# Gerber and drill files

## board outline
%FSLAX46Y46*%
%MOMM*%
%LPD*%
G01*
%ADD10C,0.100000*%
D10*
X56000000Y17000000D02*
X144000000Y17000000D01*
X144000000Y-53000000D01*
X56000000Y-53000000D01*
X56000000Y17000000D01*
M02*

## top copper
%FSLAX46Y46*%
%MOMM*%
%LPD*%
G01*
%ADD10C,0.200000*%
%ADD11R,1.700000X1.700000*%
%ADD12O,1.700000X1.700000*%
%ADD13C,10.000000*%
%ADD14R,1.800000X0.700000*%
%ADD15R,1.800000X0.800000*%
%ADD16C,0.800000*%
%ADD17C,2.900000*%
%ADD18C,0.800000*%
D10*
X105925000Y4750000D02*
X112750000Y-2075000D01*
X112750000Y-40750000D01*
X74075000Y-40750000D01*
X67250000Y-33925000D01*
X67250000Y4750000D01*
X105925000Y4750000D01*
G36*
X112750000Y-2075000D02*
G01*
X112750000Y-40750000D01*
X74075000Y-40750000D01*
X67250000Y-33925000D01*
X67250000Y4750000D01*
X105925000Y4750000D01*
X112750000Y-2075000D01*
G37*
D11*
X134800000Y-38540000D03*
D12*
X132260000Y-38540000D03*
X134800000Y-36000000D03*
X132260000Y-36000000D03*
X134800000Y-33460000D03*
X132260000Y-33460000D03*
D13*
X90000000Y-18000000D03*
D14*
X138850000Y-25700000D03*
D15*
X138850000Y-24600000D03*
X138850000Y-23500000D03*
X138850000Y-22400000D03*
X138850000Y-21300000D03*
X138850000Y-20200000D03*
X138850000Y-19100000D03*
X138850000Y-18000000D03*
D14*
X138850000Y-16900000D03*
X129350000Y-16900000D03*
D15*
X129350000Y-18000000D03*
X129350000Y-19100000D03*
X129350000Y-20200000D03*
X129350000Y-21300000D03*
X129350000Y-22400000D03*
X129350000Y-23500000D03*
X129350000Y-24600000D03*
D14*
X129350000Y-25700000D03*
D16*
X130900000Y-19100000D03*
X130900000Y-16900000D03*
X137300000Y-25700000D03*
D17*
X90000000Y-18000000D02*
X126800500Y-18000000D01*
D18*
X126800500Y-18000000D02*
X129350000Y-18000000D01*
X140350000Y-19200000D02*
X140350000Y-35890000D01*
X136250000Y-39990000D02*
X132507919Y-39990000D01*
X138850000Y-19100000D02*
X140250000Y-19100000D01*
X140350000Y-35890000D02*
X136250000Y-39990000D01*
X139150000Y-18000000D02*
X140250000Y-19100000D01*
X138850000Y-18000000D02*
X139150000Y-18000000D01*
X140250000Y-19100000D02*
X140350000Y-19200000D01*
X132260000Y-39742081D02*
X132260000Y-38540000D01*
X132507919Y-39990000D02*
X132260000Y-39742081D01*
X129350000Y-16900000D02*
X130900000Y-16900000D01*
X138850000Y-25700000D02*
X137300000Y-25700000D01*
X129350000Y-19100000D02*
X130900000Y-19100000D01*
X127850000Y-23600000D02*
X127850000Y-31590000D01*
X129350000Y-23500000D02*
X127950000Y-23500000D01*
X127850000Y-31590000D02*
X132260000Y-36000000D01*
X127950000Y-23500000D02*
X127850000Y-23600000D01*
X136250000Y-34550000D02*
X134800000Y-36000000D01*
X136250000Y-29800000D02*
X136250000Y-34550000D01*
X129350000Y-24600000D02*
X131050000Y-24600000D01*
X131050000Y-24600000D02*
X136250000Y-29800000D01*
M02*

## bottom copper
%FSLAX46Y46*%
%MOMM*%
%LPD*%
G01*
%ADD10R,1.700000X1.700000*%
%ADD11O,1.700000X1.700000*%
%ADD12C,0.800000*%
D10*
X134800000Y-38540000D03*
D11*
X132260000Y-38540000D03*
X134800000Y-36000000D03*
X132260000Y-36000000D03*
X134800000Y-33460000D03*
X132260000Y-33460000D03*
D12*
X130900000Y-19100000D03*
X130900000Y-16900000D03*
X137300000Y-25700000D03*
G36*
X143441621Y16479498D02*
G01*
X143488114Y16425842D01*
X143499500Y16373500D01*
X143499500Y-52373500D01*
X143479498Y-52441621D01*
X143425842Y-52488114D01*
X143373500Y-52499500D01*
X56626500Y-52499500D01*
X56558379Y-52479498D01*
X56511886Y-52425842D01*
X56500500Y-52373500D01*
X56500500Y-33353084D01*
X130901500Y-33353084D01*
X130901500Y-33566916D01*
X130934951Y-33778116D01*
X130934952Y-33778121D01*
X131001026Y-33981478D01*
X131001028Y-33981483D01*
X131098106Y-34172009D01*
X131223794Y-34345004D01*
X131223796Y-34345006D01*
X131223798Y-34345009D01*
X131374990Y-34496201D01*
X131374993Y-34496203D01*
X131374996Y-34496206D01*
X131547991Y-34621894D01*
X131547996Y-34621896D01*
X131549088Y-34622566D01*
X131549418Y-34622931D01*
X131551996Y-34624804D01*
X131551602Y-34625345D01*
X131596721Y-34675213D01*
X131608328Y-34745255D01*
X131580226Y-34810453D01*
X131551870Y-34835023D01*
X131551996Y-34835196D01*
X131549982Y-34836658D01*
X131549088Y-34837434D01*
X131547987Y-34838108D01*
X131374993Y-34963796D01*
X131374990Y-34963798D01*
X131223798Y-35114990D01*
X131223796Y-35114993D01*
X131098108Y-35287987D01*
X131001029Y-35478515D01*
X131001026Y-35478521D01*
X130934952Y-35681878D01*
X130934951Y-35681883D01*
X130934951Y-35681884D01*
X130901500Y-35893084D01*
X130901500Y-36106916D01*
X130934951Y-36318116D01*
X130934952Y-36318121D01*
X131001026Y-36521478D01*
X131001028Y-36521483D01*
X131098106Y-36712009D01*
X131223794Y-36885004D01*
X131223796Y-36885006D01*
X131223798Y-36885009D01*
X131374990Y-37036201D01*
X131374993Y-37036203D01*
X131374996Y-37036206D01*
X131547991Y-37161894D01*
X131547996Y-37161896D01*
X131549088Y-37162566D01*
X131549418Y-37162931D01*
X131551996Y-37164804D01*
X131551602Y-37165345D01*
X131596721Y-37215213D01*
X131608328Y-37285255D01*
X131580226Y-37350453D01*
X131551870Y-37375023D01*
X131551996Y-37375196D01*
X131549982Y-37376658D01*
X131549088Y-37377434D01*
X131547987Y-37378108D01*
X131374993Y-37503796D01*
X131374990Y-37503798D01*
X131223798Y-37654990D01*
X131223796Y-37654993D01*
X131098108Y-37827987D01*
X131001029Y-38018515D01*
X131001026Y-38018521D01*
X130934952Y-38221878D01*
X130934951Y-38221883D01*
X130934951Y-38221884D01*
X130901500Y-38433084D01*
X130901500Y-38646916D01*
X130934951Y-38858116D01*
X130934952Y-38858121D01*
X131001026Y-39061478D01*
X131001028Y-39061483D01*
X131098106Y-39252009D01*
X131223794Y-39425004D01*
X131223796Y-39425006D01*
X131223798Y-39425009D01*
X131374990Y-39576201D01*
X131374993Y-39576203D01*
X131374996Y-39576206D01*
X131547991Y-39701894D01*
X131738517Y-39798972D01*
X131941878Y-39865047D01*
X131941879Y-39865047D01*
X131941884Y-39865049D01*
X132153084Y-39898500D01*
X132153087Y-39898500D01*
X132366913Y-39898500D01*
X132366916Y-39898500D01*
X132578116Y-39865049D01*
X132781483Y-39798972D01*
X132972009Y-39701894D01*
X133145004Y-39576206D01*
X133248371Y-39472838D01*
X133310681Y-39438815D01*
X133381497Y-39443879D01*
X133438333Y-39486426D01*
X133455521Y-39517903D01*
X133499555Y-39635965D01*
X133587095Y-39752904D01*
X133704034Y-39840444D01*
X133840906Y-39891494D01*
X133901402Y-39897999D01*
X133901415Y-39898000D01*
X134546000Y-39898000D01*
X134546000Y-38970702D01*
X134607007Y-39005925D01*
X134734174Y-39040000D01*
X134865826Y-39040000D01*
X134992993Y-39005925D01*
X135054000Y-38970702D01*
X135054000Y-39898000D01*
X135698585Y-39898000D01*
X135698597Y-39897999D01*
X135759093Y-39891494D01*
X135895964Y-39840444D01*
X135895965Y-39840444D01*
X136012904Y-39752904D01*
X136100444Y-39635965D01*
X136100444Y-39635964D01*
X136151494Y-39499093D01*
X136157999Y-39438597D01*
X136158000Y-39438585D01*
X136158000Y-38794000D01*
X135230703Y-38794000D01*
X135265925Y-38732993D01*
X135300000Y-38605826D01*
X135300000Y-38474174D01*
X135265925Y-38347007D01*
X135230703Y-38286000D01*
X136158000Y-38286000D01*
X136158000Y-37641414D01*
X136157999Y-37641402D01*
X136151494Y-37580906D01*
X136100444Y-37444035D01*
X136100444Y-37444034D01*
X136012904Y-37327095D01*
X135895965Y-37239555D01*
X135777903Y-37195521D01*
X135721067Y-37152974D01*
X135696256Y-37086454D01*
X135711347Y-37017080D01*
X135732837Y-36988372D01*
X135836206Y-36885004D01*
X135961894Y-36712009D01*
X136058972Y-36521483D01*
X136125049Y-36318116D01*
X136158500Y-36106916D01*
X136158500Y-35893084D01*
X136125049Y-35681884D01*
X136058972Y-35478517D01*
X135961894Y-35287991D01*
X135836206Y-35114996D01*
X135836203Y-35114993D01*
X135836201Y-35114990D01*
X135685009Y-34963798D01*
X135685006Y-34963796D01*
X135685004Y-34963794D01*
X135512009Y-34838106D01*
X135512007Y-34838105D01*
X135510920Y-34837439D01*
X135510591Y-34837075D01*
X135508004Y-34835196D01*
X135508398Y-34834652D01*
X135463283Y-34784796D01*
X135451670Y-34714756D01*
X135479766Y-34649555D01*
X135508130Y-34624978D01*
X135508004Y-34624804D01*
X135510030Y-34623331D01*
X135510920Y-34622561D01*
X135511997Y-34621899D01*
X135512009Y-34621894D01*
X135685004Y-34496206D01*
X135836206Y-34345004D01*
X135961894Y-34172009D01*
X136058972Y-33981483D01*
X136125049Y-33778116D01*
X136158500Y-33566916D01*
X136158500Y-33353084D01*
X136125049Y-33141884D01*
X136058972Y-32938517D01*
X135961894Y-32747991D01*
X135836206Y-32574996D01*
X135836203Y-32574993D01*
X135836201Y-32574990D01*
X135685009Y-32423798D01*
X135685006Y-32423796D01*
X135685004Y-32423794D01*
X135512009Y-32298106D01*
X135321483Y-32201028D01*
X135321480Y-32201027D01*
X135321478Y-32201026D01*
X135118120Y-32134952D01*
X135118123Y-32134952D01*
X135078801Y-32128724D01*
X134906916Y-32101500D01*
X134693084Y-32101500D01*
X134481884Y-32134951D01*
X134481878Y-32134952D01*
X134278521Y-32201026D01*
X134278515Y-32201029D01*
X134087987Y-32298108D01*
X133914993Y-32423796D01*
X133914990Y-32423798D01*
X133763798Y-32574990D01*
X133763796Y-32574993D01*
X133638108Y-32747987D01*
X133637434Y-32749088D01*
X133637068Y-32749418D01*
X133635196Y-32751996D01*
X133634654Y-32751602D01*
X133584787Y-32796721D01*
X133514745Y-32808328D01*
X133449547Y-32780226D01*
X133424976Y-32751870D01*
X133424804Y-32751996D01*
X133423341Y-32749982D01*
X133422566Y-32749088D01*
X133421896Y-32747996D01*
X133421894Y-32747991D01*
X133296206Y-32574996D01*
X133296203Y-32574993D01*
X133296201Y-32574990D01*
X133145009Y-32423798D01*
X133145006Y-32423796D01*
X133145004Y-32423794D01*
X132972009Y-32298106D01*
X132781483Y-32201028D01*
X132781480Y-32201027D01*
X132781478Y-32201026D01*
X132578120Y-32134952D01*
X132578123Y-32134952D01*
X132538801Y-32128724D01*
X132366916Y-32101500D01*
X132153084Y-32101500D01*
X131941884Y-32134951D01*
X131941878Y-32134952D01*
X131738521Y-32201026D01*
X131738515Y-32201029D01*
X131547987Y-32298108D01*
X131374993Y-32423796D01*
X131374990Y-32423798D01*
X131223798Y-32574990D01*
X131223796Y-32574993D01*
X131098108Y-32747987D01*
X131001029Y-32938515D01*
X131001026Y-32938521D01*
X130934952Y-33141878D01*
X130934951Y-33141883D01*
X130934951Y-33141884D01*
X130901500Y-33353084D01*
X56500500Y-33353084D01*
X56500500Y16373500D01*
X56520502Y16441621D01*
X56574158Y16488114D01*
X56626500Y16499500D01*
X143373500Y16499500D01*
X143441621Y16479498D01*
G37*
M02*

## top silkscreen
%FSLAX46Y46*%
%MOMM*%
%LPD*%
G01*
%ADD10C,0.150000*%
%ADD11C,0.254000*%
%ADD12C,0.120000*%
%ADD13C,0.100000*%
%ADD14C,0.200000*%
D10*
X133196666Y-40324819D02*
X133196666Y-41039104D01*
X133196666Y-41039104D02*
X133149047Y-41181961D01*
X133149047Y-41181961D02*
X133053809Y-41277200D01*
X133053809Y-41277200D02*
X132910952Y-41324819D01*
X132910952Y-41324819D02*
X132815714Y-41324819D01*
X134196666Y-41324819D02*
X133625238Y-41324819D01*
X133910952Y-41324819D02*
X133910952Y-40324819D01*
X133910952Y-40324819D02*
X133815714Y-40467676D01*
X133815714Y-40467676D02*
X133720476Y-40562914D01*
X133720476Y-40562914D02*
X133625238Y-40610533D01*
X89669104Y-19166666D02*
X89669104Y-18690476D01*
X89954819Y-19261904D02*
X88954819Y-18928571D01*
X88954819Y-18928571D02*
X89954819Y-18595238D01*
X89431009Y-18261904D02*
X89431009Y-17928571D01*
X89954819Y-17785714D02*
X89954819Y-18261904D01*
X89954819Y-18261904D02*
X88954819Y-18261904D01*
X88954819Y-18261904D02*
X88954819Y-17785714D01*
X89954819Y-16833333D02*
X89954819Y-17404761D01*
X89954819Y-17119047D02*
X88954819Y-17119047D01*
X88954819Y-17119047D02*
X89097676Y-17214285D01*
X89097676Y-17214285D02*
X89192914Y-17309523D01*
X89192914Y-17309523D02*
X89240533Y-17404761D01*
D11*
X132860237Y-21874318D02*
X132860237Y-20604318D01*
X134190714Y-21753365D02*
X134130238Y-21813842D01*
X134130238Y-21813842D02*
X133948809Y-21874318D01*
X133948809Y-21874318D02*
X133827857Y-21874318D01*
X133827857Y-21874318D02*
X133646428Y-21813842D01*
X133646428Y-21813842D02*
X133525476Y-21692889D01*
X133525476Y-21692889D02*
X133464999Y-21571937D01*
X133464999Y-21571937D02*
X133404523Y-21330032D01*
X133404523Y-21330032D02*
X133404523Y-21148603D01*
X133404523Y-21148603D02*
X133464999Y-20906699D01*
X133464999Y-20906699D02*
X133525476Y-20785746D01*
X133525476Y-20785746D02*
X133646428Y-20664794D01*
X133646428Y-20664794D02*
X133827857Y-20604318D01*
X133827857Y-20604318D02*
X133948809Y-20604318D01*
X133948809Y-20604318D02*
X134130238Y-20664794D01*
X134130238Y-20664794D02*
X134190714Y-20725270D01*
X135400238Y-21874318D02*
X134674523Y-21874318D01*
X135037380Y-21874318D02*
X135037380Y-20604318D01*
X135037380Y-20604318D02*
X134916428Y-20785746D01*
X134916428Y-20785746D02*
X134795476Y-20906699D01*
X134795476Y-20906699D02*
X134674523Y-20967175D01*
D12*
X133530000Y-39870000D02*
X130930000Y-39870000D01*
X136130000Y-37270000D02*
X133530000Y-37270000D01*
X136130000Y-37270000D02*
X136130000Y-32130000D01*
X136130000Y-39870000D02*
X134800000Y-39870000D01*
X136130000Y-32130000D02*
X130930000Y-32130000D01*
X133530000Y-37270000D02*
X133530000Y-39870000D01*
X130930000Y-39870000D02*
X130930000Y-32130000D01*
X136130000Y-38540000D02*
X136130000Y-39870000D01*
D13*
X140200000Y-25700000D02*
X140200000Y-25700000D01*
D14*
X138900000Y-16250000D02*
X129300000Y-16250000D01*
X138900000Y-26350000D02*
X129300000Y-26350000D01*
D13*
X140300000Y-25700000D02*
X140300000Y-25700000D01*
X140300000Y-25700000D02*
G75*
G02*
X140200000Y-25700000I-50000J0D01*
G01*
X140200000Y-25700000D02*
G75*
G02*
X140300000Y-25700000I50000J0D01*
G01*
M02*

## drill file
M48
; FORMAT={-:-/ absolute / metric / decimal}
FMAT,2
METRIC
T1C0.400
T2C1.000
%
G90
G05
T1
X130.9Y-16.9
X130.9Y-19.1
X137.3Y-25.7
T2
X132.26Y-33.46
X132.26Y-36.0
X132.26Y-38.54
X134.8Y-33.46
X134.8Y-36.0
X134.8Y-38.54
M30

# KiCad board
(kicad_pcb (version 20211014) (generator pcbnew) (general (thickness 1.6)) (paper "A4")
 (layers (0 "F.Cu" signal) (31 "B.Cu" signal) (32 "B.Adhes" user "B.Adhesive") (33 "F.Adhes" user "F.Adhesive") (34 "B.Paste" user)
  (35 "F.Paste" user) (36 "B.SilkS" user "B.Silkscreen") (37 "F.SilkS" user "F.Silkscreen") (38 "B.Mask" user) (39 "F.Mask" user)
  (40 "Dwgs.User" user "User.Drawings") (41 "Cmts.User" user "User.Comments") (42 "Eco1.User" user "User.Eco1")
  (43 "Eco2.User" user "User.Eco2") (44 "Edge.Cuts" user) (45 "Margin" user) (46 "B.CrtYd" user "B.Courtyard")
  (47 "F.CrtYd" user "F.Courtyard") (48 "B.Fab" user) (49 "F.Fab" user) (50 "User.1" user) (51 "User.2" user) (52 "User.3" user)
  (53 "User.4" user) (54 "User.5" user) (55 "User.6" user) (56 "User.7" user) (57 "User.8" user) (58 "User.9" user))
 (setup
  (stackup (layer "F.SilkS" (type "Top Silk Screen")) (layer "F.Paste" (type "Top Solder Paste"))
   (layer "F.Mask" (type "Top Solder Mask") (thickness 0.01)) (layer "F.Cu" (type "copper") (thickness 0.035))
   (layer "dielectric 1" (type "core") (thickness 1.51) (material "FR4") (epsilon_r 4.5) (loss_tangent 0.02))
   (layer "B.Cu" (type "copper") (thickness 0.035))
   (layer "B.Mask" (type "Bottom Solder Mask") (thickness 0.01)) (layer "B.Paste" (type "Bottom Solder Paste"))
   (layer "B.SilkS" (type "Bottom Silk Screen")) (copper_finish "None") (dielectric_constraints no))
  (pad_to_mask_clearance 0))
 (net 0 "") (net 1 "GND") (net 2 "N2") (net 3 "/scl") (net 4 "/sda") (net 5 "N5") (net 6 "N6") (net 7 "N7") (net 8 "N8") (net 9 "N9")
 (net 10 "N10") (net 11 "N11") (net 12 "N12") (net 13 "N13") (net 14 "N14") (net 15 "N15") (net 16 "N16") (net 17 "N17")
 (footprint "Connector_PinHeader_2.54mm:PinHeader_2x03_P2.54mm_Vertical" (layer "F.Cu") (at 134.8 38.54 180)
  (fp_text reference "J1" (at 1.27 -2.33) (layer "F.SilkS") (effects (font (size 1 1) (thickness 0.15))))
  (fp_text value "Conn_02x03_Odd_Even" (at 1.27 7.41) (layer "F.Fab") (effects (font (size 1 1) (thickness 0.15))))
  (fp_line (start 1.27 -1.33) (end 3.87 -1.33) (layer "F.SilkS") (width 0.12))
  (fp_line (start -1.33 1.27) (end 1.27 1.27) (layer "F.SilkS") (width 0.12))
  (fp_line (start -1.33 1.27) (end -1.33 6.41) (layer "F.SilkS") (width 0.12))
  (fp_line (start -1.33 -1.33) (end 0 -1.33) (layer "F.SilkS") (width 0.12))
  (fp_line (start -1.33 6.41) (end 3.87 6.41) (layer "F.SilkS") (width 0.12))
  (fp_line (start 1.27 1.27) (end 1.27 -1.33) (layer "F.SilkS") (width 0.12))
  (fp_line (start 3.87 -1.33) (end 3.87 6.41) (layer "F.SilkS") (width 0.12))
  (fp_line (start -1.33 0) (end -1.33 -1.33) (layer "F.SilkS") (width 0.12))
  (pad "1" thru_hole rect (at 0 0 180) (size 1.7 1.7) (drill 1) (layers *.Cu *.Mask) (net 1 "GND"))
  (pad "2" thru_hole oval (at 2.54 0 180) (size 1.7 1.7) (drill 1) (layers *.Cu *.Mask) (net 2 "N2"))
  (pad "3" thru_hole oval (at 0 2.54 180) (size 1.7 1.7) (drill 1) (layers *.Cu *.Mask) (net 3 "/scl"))
  (pad "4" thru_hole oval (at 2.54 2.54 180) (size 1.7 1.7) (drill 1) (layers *.Cu *.Mask) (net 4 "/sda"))
  (pad "5" thru_hole oval (at 0 5.08 180) (size 1.7 1.7) (drill 1) (layers *.Cu *.Mask) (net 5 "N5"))
  (pad "6" thru_hole oval (at 2.54 5.08 180) (size 1.7 1.7) (drill 1) (layers *.Cu *.Mask) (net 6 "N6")))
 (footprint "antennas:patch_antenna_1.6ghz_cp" (layer "F.Cu") (at 90 18 90)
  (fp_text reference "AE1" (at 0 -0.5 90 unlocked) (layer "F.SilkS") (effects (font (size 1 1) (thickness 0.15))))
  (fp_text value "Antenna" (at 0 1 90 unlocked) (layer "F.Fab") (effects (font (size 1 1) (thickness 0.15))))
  (fp_poly
   (pts (xy 22.75 15.925) (xy 15.925 22.75) (xy -22.75 22.75) (xy -22.75 -15.925) (xy -15.925 -22.75) (xy 22.75 -22.75)) (layer "F.Cu")
   (width 0.2) (fill solid))
  (pad "1" smd circle (at 0 0 90) (size 10 10) (layers "F.Cu") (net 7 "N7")))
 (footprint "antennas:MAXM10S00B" (layer "F.Cu") (at 134.1 21.3)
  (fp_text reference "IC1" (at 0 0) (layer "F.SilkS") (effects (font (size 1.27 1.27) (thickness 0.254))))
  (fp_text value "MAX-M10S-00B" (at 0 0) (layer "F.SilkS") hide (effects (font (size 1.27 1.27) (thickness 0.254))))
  (fp_line (start 6.1 4.4) (end 6.1 4.4) (layer "F.SilkS") (width 0.1))
  (fp_line (start 4.8 -5.05) (end -4.8 -5.05) (layer "F.SilkS") (width 0.2))
  (fp_line (start 4.8 5.05) (end -4.8 5.05) (layer "F.SilkS") (width 0.2))
  (fp_line (start 6.2 4.4) (end 6.2 4.4) (layer "F.SilkS") (width 0.1))
  (fp_arc (start 6.2 4.4) (mid 6.15 4.45) (end 6.1 4.4) (layer "F.SilkS") (width 0.1))
  (fp_arc (start 6.1 4.4) (mid 6.15 4.35) (end 6.2 4.4) (layer "F.SilkS") (width 0.1))
  (pad "1" smd rect (at 4.75 4.4 90) (size 0.7 1.8) (layers "F.Cu" "F.Paste" "F.Mask") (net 1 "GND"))
  (pad "2" smd rect (at 4.75 3.3 90) (size 0.8 1.8) (layers "F.Cu" "F.Paste" "F.Mask") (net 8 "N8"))
  (pad "3" smd rect (at 4.75 2.2 90) (size 0.8 1.8) (layers "F.Cu" "F.Paste" "F.Mask") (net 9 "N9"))
  (pad "4" smd rect (at 4.75 1.1 90) (size 0.8 1.8) (layers "F.Cu" "F.Paste" "F.Mask") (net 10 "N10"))
  (pad "5" smd rect (at 4.75 0 90) (size 0.8 1.8) (layers "F.Cu" "F.Paste" "F.Mask") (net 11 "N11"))
  (pad "6" smd rect (at 4.75 -1.1 90) (size 0.8 1.8) (layers "F.Cu" "F.Paste" "F.Mask") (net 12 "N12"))
  (pad "7" smd rect (at 4.75 -2.2 90) (size 0.8 1.8) (layers "F.Cu" "F.Paste" "F.Mask") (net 2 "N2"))
  (pad "8" smd rect (at 4.75 -3.3 90) (size 0.8 1.8) (layers "F.Cu" "F.Paste" "F.Mask") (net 2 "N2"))
  (pad "9" smd rect (at 4.75 -4.4 90) (size 0.7 1.8) (layers "F.Cu" "F.Paste" "F.Mask") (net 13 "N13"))
  (pad "10" smd rect (at -4.75 -4.4 90) (size 0.7 1.8) (layers "F.Cu" "F.Paste" "F.Mask") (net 1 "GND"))
  (pad "11" smd rect (at -4.75 -3.3 90) (size 0.8 1.8) (layers "F.Cu" "F.Paste" "F.Mask") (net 7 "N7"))
  (pad "12" smd rect (at -4.75 -2.2 90) (size 0.8 1.8) (layers "F.Cu" "F.Paste" "F.Mask") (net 1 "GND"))
  (pad "13" smd rect (at -4.75 -1.1 90) (size 0.8 1.8) (layers "F.Cu" "F.Paste" "F.Mask") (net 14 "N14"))
  (pad "14" smd rect (at -4.75 0 90) (size 0.8 1.8) (layers "F.Cu" "F.Paste" "F.Mask") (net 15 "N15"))
  (pad "15" smd rect (at -4.75 1.1 90) (size 0.8 1.8) (layers "F.Cu" "F.Paste" "F.Mask") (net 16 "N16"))
  (pad "16" smd rect (at -4.75 2.2 90) (size 0.8 1.8) (layers "F.Cu" "F.Paste" "F.Mask") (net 4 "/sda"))
  (pad "17" smd rect (at -4.75 3.3 90) (size 0.8 1.8) (layers "F.Cu" "F.Paste" "F.Mask") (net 3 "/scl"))
  (pad "18" smd rect (at -4.75 4.4 90) (size 0.7 1.8) (layers "F.Cu" "F.Paste" "F.Mask") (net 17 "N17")))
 (gr_rect (start 56 -17) (end 144 53) (layer "Edge.Cuts") (width 0.1) (fill none))
 (segment (start 90 18) (end 126.8005 18) (width 2.9) (layer "F.Cu") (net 7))
 (segment (start 126.8005 18) (end 129.35 18) (width 0.8) (layer "F.Cu") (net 7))
 (segment (start 140.35 19.2) (end 140.35 35.89) (width 0.8) (layer "F.Cu") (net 2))
 (segment (start 136.25 39.99) (end 132.507919 39.99) (width 0.8) (layer "F.Cu") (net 2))
 (segment (start 138.85 19.1) (end 140.25 19.1) (width 0.8) (layer "F.Cu") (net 2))
 (segment (start 140.35 35.89) (end 136.25 39.99) (width 0.8) (layer "F.Cu") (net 2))
 (segment (start 139.15 18) (end 140.25 19.1) (width 0.8) (layer "F.Cu") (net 2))
 (segment (start 138.85 18) (end 139.15 18) (width 0.8) (layer "F.Cu") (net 2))
 (segment (start 140.25 19.1) (end 140.35 19.2) (width 0.8) (layer "F.Cu") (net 2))
 (segment (start 132.26 39.742081) (end 132.26 38.54) (width 0.8) (layer "F.Cu") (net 2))
 (segment (start 132.507919 39.99) (end 132.26 39.742081) (width 0.8) (layer "F.Cu") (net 2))
 (segment (start 129.35 16.9) (end 130.9 16.9) (width 0.8) (layer "F.Cu") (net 1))
 (segment (start 138.85 25.7) (end 137.3 25.7) (width 0.8) (layer "F.Cu") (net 1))
 (segment (start 129.35 19.1) (end 130.9 19.1) (width 0.8) (layer "F.Cu") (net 1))
 (via (at 130.9 19.1) (size 0.8) (drill 0.4) (layers "F.Cu" "B.Cu") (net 1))
 (via (at 130.9 16.9) (size 0.8) (drill 0.4) (layers "F.Cu" "B.Cu") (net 1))
 (via (at 137.3 25.7) (size 0.8) (drill 0.4) (layers "F.Cu" "B.Cu") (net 1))
 (segment (start 127.85 23.6) (end 127.85 31.59) (width 0.8) (layer "F.Cu") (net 4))
 (segment (start 129.35 23.5) (end 127.95 23.5) (width 0.8) (layer "F.Cu") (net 4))
 (segment (start 127.85 31.59) (end 132.26 36) (width 0.8) (layer "F.Cu") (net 4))
 (segment (start 127.95 23.5) (end 127.85 23.6) (width 0.8) (layer "F.Cu") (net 4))
 (segment (start 136.25 34.55) (end 134.8 36) (width 0.8) (layer "F.Cu") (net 3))
 (segment (start 136.25 29.8) (end 136.25 34.55) (width 0.8) (layer "F.Cu") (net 3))
 (segment (start 129.35 24.6) (end 131.05 24.6) (width 0.8) (layer "F.Cu") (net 3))
 (segment (start 131.05 24.6) (end 136.25 29.8) (width 0.8) (layer "F.Cu") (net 3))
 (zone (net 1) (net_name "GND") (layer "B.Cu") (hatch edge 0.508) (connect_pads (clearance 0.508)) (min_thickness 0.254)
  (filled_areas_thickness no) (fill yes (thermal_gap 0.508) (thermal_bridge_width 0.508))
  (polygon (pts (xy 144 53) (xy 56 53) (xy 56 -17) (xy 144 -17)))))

